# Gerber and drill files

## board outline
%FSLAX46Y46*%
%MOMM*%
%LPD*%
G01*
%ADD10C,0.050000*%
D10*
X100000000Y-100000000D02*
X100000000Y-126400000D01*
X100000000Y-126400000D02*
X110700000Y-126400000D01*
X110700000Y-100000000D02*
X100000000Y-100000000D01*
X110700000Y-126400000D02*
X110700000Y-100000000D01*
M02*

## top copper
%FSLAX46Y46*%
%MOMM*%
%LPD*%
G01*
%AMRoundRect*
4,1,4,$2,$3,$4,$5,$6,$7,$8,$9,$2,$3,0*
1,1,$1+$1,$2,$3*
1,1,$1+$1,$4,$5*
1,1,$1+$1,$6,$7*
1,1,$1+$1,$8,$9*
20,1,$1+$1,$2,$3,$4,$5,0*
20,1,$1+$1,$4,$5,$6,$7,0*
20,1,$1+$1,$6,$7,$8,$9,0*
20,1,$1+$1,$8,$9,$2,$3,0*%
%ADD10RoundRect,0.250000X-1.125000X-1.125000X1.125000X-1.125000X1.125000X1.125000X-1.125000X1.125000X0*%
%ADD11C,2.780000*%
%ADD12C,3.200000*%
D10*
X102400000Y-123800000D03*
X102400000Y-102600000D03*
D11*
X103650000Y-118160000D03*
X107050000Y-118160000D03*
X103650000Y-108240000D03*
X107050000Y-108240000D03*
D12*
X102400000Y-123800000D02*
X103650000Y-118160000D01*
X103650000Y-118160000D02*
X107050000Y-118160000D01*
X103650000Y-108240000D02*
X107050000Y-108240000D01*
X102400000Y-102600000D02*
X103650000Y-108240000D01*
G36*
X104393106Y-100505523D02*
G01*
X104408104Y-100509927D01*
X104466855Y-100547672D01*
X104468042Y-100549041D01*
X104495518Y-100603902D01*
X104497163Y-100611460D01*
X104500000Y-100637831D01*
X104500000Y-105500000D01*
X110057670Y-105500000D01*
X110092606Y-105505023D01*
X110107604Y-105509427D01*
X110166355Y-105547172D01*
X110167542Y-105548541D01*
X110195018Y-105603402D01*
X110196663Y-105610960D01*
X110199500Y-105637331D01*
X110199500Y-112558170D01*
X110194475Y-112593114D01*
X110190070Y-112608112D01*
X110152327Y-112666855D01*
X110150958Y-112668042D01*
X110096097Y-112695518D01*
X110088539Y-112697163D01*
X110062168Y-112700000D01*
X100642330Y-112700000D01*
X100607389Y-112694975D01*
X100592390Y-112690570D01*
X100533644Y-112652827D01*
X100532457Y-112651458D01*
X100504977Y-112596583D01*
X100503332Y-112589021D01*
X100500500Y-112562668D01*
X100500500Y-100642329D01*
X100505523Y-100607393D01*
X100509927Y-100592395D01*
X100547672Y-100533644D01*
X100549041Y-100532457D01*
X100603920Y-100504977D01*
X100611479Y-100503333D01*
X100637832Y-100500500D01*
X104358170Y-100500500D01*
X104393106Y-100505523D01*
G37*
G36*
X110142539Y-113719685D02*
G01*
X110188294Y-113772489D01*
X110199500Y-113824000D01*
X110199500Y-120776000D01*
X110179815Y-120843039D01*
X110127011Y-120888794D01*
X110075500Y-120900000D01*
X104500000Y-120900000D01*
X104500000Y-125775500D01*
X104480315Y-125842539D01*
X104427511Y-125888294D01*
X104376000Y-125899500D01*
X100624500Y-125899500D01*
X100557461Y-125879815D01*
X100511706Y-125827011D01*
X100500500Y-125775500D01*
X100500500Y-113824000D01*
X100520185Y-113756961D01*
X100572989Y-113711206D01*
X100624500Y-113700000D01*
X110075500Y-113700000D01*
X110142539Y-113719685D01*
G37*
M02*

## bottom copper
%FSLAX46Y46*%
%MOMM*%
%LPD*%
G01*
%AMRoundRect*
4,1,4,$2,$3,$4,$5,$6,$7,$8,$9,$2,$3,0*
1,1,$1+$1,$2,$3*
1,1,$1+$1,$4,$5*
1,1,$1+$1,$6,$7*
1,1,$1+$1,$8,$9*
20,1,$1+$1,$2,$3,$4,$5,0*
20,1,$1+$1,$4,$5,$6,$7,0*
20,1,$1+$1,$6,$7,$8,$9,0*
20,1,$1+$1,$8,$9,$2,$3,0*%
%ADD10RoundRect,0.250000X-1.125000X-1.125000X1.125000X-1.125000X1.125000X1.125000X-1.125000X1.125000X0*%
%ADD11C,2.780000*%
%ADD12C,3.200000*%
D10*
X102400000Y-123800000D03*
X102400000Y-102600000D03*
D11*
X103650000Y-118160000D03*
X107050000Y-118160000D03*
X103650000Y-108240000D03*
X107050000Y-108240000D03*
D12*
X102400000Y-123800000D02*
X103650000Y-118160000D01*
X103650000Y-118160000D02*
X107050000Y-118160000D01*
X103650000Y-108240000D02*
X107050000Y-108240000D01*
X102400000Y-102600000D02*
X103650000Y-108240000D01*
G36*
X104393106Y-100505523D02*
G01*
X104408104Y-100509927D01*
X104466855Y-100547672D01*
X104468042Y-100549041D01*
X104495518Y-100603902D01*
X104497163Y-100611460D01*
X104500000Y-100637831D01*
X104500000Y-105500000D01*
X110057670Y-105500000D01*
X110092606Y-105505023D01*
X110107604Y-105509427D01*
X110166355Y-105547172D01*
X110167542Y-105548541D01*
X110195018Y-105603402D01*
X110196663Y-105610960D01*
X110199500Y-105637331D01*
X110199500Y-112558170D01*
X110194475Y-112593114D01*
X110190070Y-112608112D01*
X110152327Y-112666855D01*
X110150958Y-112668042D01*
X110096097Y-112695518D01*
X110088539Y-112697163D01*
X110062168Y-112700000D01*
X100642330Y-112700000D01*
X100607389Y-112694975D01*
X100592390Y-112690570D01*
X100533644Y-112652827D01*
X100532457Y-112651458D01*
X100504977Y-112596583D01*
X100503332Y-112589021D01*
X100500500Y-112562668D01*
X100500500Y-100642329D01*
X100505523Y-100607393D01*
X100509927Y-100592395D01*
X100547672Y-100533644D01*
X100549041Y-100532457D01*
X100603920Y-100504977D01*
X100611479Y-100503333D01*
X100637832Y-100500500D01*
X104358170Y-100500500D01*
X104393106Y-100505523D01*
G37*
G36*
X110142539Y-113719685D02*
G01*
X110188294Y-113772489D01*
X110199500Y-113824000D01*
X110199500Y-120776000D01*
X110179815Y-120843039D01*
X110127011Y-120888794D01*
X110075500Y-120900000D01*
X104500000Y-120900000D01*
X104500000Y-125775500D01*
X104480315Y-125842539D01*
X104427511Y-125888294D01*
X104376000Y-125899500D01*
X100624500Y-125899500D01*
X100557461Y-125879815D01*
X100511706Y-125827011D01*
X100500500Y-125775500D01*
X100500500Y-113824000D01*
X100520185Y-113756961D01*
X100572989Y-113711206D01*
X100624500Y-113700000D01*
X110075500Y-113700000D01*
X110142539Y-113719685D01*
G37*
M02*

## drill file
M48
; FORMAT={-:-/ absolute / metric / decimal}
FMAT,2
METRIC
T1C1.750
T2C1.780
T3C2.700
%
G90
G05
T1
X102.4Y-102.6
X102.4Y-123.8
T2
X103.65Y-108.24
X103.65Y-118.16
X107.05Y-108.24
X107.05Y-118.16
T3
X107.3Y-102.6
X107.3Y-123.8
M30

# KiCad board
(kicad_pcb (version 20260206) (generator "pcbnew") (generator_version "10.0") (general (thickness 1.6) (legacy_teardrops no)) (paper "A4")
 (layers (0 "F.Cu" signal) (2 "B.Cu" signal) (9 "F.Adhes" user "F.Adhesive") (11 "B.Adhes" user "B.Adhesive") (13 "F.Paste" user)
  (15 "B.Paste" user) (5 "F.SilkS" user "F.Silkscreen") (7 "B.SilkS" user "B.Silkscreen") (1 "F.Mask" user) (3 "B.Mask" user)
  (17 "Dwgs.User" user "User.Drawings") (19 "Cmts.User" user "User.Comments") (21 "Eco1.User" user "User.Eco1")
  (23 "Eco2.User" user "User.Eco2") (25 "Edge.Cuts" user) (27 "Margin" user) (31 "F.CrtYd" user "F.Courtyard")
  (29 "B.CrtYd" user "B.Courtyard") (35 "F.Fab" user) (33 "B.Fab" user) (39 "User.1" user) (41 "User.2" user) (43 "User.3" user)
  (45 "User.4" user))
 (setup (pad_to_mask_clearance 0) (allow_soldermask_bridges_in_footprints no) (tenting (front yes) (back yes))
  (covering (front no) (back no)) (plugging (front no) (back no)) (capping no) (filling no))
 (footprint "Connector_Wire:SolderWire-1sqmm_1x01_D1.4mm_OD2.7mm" (layer "F.Cu") (at 102.4 123.8)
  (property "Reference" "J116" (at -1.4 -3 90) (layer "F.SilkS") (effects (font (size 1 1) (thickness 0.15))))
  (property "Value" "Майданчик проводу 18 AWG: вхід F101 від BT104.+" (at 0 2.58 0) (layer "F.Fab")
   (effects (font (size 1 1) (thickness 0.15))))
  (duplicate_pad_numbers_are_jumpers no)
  (pad "1" thru_hole roundrect (at 0 0) (size 2.75 2.75) (drill 1.75) (layers "*.Cu" "*.Mask") (remove_unused_layers no)
   (roundrect_rratio 0.090909) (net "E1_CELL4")))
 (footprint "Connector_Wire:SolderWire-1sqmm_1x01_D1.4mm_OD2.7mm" (layer "F.Cu") (at 102.4 102.6)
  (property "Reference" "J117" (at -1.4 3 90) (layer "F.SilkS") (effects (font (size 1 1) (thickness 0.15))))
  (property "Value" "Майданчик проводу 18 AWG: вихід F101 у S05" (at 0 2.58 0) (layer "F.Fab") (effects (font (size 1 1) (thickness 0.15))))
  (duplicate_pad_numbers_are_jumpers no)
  (pad "1" thru_hole roundrect (at 0 0) (size 2.75 2.75) (drill 1.75) (layers "*.Cu" "*.Mask") (remove_unused_layers no)
   (roundrect_rratio 0.090909) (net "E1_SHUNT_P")))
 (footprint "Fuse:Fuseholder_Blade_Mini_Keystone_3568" (layer "F.Cu") (at 103.65 118.16 90)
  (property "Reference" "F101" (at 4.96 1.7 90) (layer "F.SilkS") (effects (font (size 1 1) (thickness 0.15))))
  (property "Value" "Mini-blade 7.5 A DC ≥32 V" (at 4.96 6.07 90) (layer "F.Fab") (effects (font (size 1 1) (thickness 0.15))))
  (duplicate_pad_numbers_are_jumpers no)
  (pad "1" thru_hole circle (at 0 0 90) (size 2.78 2.78) (drill 1.78) (layers "*.Cu" "*.Mask") (remove_unused_layers no) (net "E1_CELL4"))
  (pad "1" thru_hole circle (at 0 3.4 90) (size 2.78 2.78) (drill 1.78) (layers "*.Cu" "*.Mask") (remove_unused_layers no) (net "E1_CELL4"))
  (pad "2" thru_hole circle (at 9.92 0 90) (size 2.78 2.78) (drill 1.78) (layers "*.Cu" "*.Mask") (remove_unused_layers no)
   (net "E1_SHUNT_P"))
  (pad "2" thru_hole circle (at 9.92 3.4 90) (size 2.78 2.78) (drill 1.78) (layers "*.Cu" "*.Mask") (remove_unused_layers no)
   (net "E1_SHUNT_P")))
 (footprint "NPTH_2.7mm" (layer "F.Cu") (at 107.3 123.8)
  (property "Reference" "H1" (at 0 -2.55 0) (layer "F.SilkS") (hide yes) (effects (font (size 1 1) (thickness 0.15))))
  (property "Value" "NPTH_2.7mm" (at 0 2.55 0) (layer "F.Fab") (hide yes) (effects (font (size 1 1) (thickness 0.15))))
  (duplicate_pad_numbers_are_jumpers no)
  (pad "" np_thru_hole circle (at 0 0) (size 2.7 2.7) (drill 2.7) (layers "*.Cu" "*.Mask")))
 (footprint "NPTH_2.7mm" (layer "F.Cu") (at 107.3 102.6)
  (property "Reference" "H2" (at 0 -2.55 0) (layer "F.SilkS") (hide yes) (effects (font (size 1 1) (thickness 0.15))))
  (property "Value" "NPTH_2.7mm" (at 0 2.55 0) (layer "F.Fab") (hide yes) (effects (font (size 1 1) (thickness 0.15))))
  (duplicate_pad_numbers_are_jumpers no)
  (pad "" np_thru_hole circle (at 0 0) (size 2.7 2.7) (drill 2.7) (layers "*.Cu" "*.Mask")))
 (gr_line (start 100 100) (end 100 126.4) (stroke (width 0.05) (type default)) (layer "Edge.Cuts"))
 (gr_line (start 100 126.4) (end 110.7 126.4) (stroke (width 0.05) (type default)) (layer "Edge.Cuts"))
 (gr_line (start 110.7 100) (end 100 100) (stroke (width 0.05) (type default)) (layer "Edge.Cuts"))
 (gr_line (start 110.7 126.4) (end 110.7 100) (stroke (width 0.05) (type default)) (layer "Edge.Cuts"))
 (segment (start 102.4 123.8) (end 103.65 118.16) (width 3.2) (locked yes) (layer "F.Cu") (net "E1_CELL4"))
 (segment (start 103.65 118.16) (end 107.05 118.16) (width 3.2) (locked yes) (layer "F.Cu") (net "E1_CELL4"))
 (segment (start 102.4 123.8) (end 103.65 118.16) (width 3.2) (locked yes) (layer "B.Cu") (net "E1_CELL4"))
 (segment (start 103.65 118.16) (end 107.05 118.16) (width 3.2) (locked yes) (layer "B.Cu") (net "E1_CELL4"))
 (segment (start 103.65 108.24) (end 107.05 108.24) (width 3.2) (locked yes) (layer "F.Cu") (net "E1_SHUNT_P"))
 (segment (start 102.4 102.6) (end 103.65 108.24) (width 3.2) (locked yes) (layer "F.Cu") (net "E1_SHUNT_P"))
 (segment (start 103.65 108.24) (end 107.05 108.24) (width 3.2) (locked yes) (layer "B.Cu") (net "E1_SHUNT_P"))
 (segment (start 102.4 102.6) (end 103.65 108.24) (width 3.2) (locked yes) (layer "B.Cu") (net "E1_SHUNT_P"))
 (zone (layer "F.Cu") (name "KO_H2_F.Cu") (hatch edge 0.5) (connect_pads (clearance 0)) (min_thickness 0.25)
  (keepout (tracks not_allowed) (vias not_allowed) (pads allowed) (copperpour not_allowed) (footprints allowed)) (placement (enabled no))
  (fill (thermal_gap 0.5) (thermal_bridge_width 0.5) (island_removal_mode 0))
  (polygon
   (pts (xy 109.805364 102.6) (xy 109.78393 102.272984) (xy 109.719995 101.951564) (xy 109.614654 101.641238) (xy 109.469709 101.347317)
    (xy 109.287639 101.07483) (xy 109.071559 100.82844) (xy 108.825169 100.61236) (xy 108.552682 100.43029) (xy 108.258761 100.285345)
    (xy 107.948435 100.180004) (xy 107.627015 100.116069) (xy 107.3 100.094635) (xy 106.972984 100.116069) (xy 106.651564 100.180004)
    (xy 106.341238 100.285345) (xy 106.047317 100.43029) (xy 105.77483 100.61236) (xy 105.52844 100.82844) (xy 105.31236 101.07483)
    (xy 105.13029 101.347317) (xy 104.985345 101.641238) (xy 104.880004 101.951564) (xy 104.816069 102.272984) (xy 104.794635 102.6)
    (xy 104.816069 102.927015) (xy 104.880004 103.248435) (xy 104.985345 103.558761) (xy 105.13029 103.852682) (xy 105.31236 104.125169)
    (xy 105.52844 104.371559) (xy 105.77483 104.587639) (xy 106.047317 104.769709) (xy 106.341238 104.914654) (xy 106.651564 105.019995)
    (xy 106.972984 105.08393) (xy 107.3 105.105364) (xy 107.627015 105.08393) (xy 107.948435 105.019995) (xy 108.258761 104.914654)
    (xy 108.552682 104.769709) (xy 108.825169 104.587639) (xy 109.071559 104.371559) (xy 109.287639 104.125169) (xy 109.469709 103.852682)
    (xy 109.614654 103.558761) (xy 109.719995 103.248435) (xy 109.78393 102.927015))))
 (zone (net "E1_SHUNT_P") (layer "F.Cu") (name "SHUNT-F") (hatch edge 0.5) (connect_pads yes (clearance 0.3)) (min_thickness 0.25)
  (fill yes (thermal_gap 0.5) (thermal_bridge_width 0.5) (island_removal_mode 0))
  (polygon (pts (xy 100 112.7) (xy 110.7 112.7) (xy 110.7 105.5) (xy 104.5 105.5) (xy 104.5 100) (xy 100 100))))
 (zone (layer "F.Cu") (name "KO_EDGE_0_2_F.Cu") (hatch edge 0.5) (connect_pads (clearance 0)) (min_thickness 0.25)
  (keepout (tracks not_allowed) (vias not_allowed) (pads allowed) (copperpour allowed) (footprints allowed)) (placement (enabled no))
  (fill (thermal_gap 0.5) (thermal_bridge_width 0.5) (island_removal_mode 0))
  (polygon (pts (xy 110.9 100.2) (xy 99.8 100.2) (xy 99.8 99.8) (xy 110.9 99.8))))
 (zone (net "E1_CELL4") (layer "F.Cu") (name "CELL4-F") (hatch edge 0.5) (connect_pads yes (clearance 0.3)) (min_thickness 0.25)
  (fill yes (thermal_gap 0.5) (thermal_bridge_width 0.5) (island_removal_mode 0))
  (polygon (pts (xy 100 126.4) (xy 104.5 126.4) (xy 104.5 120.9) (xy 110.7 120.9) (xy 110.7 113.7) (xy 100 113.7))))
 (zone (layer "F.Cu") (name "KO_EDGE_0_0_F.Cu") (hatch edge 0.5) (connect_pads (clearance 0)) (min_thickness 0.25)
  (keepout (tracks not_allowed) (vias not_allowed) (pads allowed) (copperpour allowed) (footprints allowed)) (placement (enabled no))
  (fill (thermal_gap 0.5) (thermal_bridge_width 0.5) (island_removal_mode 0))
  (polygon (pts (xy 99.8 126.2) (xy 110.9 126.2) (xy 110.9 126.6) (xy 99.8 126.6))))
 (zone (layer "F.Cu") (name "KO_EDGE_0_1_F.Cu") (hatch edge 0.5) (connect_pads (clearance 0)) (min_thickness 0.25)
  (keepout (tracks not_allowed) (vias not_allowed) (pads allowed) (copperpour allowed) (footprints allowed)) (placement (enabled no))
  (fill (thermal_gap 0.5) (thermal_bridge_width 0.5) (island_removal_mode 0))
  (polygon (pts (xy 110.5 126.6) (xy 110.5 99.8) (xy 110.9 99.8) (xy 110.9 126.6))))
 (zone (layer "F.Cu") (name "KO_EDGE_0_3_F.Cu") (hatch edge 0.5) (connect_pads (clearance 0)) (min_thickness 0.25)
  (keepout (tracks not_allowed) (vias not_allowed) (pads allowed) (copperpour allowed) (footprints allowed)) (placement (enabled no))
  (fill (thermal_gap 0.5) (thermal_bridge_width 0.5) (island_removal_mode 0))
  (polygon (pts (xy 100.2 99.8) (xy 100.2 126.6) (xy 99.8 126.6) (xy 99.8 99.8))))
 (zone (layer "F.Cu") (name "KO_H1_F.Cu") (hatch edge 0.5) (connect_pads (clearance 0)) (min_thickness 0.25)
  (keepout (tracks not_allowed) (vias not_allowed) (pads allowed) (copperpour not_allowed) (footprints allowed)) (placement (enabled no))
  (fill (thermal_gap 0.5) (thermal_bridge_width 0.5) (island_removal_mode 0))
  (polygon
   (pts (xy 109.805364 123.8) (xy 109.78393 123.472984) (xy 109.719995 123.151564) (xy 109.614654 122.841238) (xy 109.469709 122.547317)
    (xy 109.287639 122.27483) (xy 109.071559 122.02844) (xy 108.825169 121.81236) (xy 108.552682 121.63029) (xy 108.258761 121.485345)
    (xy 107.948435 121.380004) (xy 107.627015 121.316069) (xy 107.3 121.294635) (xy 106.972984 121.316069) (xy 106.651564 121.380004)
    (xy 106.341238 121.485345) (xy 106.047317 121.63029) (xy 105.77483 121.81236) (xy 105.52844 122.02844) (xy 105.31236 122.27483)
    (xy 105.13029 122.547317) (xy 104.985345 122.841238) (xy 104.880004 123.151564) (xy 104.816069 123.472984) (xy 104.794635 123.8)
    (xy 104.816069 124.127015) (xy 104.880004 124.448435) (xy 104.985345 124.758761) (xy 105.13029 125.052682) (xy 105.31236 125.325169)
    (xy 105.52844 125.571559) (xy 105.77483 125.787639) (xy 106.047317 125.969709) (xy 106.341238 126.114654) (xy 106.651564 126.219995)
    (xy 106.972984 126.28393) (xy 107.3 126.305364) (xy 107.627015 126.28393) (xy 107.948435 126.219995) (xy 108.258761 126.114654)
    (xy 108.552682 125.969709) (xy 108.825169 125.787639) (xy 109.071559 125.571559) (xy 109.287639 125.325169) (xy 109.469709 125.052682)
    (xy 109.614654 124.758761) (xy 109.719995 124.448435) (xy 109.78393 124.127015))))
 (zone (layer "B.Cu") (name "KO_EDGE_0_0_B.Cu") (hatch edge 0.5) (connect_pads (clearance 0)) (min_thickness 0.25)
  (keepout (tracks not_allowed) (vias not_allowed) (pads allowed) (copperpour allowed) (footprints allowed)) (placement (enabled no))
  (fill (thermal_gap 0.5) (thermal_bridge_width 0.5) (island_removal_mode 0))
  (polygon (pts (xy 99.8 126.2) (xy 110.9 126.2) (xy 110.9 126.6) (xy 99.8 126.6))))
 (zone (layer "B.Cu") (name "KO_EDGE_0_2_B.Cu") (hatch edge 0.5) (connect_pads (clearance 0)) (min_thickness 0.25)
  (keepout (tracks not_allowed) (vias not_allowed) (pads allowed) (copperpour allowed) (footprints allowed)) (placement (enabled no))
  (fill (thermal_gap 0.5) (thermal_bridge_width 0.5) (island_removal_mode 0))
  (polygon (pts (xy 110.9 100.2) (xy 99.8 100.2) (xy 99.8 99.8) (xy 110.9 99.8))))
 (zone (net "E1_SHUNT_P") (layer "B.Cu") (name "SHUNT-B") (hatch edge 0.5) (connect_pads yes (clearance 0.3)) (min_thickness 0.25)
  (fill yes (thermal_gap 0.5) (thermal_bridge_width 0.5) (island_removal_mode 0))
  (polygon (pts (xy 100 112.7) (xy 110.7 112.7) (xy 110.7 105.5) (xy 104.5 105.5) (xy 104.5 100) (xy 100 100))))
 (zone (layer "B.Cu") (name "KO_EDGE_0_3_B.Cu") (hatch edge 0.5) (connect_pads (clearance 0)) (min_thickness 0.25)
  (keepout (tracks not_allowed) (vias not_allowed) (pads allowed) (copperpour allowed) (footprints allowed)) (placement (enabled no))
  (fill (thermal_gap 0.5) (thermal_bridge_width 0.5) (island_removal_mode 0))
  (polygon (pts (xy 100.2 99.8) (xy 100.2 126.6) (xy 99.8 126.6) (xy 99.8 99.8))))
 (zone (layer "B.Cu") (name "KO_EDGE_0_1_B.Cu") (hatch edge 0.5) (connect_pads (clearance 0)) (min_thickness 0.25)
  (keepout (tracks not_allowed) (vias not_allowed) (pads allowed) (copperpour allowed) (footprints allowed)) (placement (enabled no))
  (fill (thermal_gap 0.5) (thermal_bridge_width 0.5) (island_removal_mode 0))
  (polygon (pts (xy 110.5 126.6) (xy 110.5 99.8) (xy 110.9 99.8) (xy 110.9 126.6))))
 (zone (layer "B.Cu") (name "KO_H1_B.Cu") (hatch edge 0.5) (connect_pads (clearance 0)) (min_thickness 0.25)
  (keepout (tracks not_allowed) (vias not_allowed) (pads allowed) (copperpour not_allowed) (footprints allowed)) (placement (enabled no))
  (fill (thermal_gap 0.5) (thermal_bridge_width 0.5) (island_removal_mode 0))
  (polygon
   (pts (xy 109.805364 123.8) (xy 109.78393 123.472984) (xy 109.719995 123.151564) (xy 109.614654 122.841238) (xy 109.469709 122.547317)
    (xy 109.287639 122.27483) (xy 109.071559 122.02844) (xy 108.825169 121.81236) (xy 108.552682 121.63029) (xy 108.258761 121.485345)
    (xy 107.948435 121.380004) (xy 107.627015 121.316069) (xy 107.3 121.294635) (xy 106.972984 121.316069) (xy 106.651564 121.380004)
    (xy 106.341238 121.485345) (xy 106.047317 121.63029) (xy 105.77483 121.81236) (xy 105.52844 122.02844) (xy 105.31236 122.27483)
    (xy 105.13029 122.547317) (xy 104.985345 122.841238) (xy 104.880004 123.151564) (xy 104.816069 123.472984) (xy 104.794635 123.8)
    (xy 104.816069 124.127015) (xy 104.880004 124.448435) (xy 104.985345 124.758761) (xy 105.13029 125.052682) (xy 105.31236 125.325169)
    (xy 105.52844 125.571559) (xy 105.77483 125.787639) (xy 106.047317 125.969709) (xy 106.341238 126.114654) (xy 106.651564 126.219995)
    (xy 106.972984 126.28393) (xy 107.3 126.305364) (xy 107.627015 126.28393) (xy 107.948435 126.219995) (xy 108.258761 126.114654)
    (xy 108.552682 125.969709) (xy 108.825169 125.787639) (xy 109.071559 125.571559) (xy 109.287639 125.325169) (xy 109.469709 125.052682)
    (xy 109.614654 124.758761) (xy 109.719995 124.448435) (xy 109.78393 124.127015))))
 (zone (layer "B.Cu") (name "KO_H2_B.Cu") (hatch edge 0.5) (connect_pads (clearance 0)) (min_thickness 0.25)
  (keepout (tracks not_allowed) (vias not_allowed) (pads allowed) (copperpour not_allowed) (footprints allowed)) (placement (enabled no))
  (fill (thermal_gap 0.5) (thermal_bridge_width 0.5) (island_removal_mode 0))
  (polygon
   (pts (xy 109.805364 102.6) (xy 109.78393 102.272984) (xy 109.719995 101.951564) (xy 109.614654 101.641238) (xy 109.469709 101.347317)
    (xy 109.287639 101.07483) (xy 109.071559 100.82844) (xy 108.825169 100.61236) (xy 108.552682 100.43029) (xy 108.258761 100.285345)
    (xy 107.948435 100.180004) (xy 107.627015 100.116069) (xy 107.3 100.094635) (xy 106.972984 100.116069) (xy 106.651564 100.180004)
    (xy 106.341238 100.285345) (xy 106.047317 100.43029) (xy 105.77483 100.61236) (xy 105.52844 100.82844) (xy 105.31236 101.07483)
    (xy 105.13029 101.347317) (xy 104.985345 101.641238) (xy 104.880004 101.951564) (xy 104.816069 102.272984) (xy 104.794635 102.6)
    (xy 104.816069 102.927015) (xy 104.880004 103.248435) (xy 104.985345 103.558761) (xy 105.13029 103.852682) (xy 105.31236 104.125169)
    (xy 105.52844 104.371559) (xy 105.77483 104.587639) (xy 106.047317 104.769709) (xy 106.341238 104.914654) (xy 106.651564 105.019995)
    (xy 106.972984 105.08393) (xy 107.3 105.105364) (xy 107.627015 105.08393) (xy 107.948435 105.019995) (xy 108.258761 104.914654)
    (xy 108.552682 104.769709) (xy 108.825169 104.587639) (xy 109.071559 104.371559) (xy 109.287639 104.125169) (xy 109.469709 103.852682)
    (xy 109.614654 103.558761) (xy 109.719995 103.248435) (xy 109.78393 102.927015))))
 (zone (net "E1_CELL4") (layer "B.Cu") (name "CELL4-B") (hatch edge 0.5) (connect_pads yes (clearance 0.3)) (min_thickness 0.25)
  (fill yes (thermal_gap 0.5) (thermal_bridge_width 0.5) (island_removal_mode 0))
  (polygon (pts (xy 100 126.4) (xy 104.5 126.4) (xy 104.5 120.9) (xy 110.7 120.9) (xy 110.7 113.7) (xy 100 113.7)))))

